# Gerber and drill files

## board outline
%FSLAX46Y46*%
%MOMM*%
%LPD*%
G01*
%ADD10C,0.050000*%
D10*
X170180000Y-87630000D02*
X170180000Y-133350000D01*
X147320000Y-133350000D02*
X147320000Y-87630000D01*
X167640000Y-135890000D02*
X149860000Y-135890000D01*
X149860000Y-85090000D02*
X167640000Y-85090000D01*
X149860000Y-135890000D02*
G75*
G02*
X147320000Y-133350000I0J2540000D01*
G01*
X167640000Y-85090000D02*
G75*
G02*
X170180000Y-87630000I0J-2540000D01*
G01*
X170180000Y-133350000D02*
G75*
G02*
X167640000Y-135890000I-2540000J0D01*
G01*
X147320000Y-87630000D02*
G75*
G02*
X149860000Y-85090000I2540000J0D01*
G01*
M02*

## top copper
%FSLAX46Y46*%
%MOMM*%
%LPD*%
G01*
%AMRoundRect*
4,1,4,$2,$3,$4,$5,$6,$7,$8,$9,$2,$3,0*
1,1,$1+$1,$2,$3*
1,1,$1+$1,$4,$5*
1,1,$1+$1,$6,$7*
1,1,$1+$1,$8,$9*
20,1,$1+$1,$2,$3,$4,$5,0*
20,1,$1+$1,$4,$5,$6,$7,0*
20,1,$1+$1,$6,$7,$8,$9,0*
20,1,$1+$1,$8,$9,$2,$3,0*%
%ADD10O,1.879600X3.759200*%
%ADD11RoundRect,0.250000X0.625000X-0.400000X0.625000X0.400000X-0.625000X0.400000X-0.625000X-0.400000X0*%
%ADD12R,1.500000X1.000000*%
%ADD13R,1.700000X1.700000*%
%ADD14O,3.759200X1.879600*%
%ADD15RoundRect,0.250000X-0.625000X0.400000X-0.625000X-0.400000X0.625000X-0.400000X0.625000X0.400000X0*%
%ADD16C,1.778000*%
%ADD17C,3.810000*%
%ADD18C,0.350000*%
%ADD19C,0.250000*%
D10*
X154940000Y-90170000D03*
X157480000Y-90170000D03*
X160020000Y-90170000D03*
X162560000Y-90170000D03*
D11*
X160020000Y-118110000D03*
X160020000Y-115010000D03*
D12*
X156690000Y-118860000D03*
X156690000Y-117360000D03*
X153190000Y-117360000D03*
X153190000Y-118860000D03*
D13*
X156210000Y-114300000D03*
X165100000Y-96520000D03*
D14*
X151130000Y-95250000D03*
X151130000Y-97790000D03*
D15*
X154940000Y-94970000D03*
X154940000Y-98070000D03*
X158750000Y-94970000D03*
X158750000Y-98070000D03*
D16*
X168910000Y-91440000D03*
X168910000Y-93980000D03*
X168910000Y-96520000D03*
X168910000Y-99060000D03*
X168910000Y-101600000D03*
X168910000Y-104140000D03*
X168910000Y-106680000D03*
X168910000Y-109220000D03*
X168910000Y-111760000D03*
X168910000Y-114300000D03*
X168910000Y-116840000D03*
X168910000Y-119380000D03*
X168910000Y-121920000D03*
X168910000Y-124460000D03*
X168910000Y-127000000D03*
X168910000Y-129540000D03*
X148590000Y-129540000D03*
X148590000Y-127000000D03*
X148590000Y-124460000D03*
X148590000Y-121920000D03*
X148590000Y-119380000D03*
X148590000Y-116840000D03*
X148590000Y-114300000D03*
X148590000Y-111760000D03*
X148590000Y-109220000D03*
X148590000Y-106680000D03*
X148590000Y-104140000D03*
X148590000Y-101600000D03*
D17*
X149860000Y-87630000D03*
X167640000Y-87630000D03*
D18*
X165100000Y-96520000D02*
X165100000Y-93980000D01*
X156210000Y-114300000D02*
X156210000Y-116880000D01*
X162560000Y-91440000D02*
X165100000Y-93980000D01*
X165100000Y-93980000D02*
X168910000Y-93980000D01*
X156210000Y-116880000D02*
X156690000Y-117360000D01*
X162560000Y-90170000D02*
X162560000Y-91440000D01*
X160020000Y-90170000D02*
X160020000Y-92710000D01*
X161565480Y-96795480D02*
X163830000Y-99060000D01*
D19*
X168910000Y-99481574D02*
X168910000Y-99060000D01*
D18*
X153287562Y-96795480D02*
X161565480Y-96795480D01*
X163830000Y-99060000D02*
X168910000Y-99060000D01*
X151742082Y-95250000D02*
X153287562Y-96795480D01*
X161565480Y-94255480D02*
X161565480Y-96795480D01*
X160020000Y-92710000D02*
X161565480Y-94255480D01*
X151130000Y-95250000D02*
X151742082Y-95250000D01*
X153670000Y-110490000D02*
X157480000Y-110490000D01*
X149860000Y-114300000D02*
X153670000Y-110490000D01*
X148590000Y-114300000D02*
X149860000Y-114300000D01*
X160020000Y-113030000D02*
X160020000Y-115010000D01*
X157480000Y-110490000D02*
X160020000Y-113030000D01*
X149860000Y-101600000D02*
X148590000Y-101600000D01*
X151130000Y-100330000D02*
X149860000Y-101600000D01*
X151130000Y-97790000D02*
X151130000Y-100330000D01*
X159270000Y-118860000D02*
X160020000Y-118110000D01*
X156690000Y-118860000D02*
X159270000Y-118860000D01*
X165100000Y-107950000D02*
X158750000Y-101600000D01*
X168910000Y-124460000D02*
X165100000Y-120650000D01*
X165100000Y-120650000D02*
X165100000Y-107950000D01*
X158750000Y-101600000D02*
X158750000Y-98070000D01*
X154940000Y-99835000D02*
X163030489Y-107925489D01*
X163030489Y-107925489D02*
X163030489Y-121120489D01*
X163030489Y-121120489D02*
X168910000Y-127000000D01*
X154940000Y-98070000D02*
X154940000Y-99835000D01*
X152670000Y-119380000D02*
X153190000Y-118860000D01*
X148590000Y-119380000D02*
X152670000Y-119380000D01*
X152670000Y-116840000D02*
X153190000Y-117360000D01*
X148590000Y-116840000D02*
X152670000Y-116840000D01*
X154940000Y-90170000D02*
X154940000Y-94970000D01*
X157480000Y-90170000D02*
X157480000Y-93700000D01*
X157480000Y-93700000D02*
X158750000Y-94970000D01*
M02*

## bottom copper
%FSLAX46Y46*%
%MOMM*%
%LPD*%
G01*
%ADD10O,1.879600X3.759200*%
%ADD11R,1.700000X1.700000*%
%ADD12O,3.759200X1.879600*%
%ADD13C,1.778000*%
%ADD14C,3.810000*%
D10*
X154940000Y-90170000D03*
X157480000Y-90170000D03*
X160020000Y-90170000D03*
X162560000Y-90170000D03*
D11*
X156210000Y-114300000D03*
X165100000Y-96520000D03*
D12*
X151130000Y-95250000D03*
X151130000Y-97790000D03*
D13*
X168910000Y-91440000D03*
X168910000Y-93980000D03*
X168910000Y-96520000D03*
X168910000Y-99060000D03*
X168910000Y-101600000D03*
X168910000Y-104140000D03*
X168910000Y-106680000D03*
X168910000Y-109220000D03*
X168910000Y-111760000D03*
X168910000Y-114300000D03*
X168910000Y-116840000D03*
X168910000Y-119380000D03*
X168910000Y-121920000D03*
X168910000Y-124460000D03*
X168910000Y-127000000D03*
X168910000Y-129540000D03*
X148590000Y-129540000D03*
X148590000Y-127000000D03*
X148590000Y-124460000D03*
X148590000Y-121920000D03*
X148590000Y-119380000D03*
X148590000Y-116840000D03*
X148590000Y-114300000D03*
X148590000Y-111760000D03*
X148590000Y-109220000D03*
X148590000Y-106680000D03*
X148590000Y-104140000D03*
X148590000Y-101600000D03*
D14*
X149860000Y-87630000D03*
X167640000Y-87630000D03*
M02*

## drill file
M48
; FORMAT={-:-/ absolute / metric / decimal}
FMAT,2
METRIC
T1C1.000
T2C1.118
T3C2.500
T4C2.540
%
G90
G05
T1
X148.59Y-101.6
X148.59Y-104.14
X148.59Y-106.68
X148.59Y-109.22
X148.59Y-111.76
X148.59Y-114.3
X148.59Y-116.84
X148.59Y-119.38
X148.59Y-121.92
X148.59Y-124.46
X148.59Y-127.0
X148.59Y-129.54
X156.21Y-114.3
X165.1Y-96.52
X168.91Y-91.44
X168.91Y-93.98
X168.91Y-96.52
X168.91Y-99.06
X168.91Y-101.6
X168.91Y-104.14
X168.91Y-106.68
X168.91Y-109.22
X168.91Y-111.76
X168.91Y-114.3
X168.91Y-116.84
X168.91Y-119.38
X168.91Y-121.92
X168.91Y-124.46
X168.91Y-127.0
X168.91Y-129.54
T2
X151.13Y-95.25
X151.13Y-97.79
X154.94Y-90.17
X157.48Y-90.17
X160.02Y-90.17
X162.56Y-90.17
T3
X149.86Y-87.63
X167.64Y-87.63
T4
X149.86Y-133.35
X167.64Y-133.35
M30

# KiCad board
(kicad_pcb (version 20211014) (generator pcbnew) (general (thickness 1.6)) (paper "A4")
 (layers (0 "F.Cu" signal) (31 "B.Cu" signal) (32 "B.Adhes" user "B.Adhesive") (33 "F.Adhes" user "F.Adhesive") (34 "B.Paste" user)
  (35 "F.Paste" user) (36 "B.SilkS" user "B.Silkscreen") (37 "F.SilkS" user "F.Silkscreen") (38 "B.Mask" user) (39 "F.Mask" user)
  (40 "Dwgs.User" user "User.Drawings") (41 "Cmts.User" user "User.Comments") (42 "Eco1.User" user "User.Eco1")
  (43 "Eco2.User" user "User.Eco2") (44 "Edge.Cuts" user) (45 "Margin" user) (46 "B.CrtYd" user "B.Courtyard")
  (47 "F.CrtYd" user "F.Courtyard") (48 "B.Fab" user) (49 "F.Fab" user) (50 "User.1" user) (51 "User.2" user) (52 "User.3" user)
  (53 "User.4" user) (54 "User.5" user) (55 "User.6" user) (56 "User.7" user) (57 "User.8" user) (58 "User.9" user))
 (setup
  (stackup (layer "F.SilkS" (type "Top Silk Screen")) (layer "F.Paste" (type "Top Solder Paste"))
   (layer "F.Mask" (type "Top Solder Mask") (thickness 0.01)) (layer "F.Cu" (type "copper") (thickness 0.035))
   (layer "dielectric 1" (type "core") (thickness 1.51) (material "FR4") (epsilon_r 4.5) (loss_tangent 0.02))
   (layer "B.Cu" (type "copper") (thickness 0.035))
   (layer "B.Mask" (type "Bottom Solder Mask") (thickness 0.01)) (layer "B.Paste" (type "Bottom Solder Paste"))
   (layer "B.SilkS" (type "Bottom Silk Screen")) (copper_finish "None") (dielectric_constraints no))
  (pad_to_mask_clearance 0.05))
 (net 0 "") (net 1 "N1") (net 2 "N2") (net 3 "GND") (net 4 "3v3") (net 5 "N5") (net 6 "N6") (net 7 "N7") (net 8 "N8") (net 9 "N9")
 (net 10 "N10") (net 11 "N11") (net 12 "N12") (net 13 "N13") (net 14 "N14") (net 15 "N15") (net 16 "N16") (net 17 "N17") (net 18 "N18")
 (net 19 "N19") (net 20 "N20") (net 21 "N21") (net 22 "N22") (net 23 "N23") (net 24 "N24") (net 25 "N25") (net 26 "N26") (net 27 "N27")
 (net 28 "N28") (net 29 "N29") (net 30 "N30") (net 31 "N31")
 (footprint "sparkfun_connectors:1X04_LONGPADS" (layer "F.Cu") (at 154.94 90.17)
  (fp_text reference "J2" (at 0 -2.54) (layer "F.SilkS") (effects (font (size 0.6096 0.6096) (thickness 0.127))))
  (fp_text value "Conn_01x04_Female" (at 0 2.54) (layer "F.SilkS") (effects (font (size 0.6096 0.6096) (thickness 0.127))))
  (pad "1" thru_hole oval locked (at 0 0 180) (size 1.8796 3.7592) (drill 1.1176) (layers *.Cu *.Mask) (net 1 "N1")
   (solder_mask_margin 0.1016))
  (pad "2" thru_hole oval locked (at 2.54 0 180) (size 1.8796 3.7592) (drill 1.1176) (layers *.Cu *.Mask) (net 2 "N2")
   (solder_mask_margin 0.1016))
  (pad "3" thru_hole oval locked (at 5.08 0 180) (size 1.8796 3.7592) (drill 1.1176) (layers *.Cu *.Mask) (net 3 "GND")
   (solder_mask_margin 0.1016))
  (pad "4" thru_hole oval locked (at 7.62 0 180) (size 1.8796 3.7592) (drill 1.1176) (layers *.Cu *.Mask) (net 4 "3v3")
   (solder_mask_margin 0.1016)))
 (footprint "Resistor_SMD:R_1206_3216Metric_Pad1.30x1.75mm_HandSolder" (layer "F.Cu") (at 160.02 116.56 90)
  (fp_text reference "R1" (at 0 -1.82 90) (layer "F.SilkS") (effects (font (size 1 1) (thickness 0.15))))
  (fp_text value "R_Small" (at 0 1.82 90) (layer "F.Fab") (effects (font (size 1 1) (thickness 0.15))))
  (pad "1" smd roundrect (at -1.55 0 90) (size 1.3 1.75) (layers "F.Cu" "F.Paste" "F.Mask") (roundrect_rratio 0.192308) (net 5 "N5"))
  (pad "2" smd roundrect (at 1.55 0 90) (size 1.3 1.75) (layers "F.Cu" "F.Paste" "F.Mask") (roundrect_rratio 0.192308) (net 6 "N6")))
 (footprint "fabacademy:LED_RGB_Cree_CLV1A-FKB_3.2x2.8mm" (layer "F.Cu") (at 154.94 118.11 180)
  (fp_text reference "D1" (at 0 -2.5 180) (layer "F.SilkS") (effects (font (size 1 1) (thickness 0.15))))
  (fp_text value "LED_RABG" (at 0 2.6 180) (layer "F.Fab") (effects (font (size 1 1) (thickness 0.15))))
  (pad "1" smd rect locked (at -1.75 -0.75) (size 1.5 1) (layers "F.Cu" "F.Paste" "F.Mask") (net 5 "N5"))
  (pad "2" smd rect locked (at -1.75 0.75) (size 1.5 1) (layers "F.Cu" "F.Paste" "F.Mask") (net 4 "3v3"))
  (pad "3" smd rect locked (at 1.75 0.75) (size 1.5 1) (layers "F.Cu" "F.Paste" "F.Mask") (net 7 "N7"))
  (pad "4" smd rect locked (at 1.75 -0.75) (size 1.5 1) (layers "F.Cu" "F.Paste" "F.Mask") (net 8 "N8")))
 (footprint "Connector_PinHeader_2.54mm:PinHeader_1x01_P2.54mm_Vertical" (layer "F.Cu") (at 156.21 114.3)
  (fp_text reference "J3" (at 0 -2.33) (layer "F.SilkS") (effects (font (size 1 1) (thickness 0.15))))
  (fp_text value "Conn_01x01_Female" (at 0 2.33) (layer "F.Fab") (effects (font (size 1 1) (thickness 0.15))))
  (pad "1" thru_hole rect (at 0 0) (size 1.7 1.7) (drill 1) (layers *.Cu *.Mask) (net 4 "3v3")))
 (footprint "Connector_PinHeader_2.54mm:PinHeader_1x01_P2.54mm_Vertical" (layer "F.Cu") (at 165.1 96.52)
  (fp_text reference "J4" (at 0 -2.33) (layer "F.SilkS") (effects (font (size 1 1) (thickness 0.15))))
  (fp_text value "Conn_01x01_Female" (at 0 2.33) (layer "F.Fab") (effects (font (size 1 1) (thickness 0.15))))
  (pad "1" thru_hole rect (at 0 0) (size 1.7 1.7) (drill 1) (layers *.Cu *.Mask) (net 4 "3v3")))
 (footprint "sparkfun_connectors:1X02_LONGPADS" (layer "F.Cu") (at 151.13 95.25 -90)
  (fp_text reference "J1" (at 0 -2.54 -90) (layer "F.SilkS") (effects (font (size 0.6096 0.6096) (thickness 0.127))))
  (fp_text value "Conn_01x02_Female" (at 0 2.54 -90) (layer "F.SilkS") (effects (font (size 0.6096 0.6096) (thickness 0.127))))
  (pad "1" thru_hole oval locked (at 0 0 90) (size 1.8796 3.7592) (drill 1.1176) (layers *.Cu *.Mask) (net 3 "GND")
   (solder_mask_margin 0.1016))
  (pad "2" thru_hole oval locked (at 2.54 0 90) (size 1.8796 3.7592) (drill 1.1176) (layers *.Cu *.Mask) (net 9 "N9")
   (solder_mask_margin 0.1016)))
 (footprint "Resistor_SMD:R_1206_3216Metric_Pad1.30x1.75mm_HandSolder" (layer "F.Cu") (at 154.94 96.52 -90)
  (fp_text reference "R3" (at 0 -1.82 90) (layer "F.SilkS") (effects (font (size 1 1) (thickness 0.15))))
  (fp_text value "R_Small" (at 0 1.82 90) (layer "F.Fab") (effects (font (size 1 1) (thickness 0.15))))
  (pad "1" smd roundrect (at -1.55 0 270) (size 1.3 1.75) (layers "F.Cu" "F.Paste" "F.Mask") (roundrect_rratio 0.192308) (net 1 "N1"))
  (pad "2" smd roundrect (at 1.55 0 270) (size 1.3 1.75) (layers "F.Cu" "F.Paste" "F.Mask") (roundrect_rratio 0.192308) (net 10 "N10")))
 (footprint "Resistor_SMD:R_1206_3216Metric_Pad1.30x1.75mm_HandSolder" (layer "F.Cu") (at 158.75 96.52 -90)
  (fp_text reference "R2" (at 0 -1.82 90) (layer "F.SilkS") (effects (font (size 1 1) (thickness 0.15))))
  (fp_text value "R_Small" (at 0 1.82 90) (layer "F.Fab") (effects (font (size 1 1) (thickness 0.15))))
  (pad "1" smd roundrect (at -1.55 0 270) (size 1.3 1.75) (layers "F.Cu" "F.Paste" "F.Mask") (roundrect_rratio 0.192308) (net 2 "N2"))
  (pad "2" smd roundrect (at 1.55 0 270) (size 1.3 1.75) (layers "F.Cu" "F.Paste" "F.Mask") (roundrect_rratio 0.192308) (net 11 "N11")))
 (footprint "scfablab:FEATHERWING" (layer "B.Cu") (at 170.18 85.09 -90)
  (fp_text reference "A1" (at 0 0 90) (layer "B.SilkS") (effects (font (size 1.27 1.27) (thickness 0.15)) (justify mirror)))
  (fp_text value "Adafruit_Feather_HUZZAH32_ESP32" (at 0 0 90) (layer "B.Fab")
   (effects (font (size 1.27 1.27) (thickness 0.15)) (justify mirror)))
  (fp_line (start 2.54 0) (end 48.26 0) (layer "Edge.Cuts") (width 0.05))
  (fp_line (start 48.26 22.86) (end 2.54 22.86) (layer "Edge.Cuts") (width 0.05))
  (fp_line (start 50.8 2.54) (end 50.8 20.32) (layer "Edge.Cuts") (width 0.05))
  (fp_line (start 0 20.32) (end 0 2.54) (layer "Edge.Cuts") (width 0.05))
  (fp_arc (start 50.8 20.32) (mid 50.056051 22.116051) (end 48.26 22.86) (layer "Edge.Cuts") (width 0.05))
  (fp_arc (start 0 2.54) (mid 0.743949 0.743949) (end 2.54 0) (layer "Edge.Cuts") (width 0.05))
  (fp_arc (start 48.26 0) (mid 50.056051 0.743949) (end 50.8 2.54) (layer "Edge.Cuts") (width 0.05))
  (fp_arc (start 2.54 22.86) (mid 0.743949 22.116051) (end 0 20.32) (layer "Edge.Cuts") (width 0.05))
  (pad "" np_thru_hole circle (at 48.26 20.32 270) (size 2.54 2.54) (drill 2.54) (layers *.Cu *.Mask))
  (pad "" np_thru_hole circle (at 48.26 2.54 270) (size 2.54 2.54) (drill 2.54) (layers *.Cu *.Mask))
  (pad "1" thru_hole circle (at 6.35 1.27 270) (size 1.778 1.778) (drill 1) (layers *.Cu *.Mask) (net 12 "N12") (solder_mask_margin 0.1016))
  (pad "2" thru_hole circle (at 8.89 1.27 270) (size 1.778 1.778) (drill 1) (layers *.Cu *.Mask) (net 4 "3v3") (solder_mask_margin 0.1016))
  (pad "3" thru_hole circle (at 11.43 1.27 270) (size 1.778 1.778) (drill 1) (layers *.Cu *.Mask) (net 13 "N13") (solder_mask_margin 0.1016))
  (pad "4" thru_hole circle (at 13.97 1.27 270) (size 1.778 1.778) (drill 1) (layers *.Cu *.Mask) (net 3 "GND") (solder_mask_margin 0.1016))
  (pad "5" thru_hole circle (at 16.51 1.27 270) (size 1.778 1.778) (drill 1) (layers *.Cu *.Mask) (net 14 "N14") (solder_mask_margin 0.1016))
  (pad "6" thru_hole circle (at 19.05 1.27 270) (size 1.778 1.778) (drill 1) (layers *.Cu *.Mask) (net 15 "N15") (solder_mask_margin 0.1016))
  (pad "7" thru_hole circle (at 21.59 1.27 270) (size 1.778 1.778) (drill 1) (layers *.Cu *.Mask) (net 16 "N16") (solder_mask_margin 0.1016))
  (pad "8" thru_hole circle (at 24.13 1.27 270) (size 1.778 1.778) (drill 1) (layers *.Cu *.Mask) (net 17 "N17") (solder_mask_margin 0.1016))
  (pad "9" thru_hole circle (at 26.67 1.27 270) (size 1.778 1.778) (drill 1) (layers *.Cu *.Mask) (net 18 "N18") (solder_mask_margin 0.1016))
  (pad "10" thru_hole circle (at 29.21 1.27 270) (size 1.778 1.778) (drill 1) (layers *.Cu *.Mask) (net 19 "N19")
   (solder_mask_margin 0.1016))
  (pad "11" thru_hole circle (at 31.75 1.27 270) (size 1.778 1.778) (drill 1) (layers *.Cu *.Mask) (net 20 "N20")
   (solder_mask_margin 0.1016))
  (pad "12" thru_hole circle (at 34.29 1.27 270) (size 1.778 1.778) (drill 1) (layers *.Cu *.Mask) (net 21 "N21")
   (solder_mask_margin 0.1016))
  (pad "13" thru_hole circle (at 36.83 1.27 270) (size 1.778 1.778) (drill 1) (layers *.Cu *.Mask) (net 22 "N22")
   (solder_mask_margin 0.1016))
  (pad "14" thru_hole circle (at 39.37 1.27 270) (size 1.778 1.778) (drill 1) (layers *.Cu *.Mask) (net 11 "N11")
   (solder_mask_margin 0.1016))
  (pad "15" thru_hole circle (at 41.91 1.27 270) (size 1.778 1.778) (drill 1) (layers *.Cu *.Mask) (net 10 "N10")
   (solder_mask_margin 0.1016))
  (pad "16" thru_hole circle (at 44.45 1.27 270) (size 1.778 1.778) (drill 1) (layers *.Cu *.Mask) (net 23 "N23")
   (solder_mask_margin 0.1016))
  (pad "17" thru_hole circle (at 44.45 21.59 270) (size 1.778 1.778) (drill 1) (layers *.Cu *.Mask) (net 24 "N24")
   (solder_mask_margin 0.1016))
  (pad "18" thru_hole circle (at 41.91 21.59 270) (size 1.778 1.778) (drill 1) (layers *.Cu *.Mask) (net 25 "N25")
   (solder_mask_margin 0.1016))
  (pad "19" thru_hole circle (at 39.37 21.59 270) (size 1.778 1.778) (drill 1) (layers *.Cu *.Mask) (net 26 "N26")
   (solder_mask_margin 0.1016))
  (pad "20" thru_hole circle (at 36.83 21.59 270) (size 1.778 1.778) (drill 1) (layers *.Cu *.Mask) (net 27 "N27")
   (solder_mask_margin 0.1016))
  (pad "21" thru_hole circle (at 34.29 21.59 270) (size 1.778 1.778) (drill 1) (layers *.Cu *.Mask) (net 8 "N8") (solder_mask_margin 0.1016))
  (pad "22" thru_hole circle (at 31.75 21.59 270) (size 1.778 1.778) (drill 1) (layers *.Cu *.Mask) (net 7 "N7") (solder_mask_margin 0.1016))
  (pad "23" thru_hole circle (at 29.21 21.59 270) (size 1.778 1.778) (drill 1) (layers *.Cu *.Mask) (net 6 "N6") (solder_mask_margin 0.1016))
  (pad "24" thru_hole circle (at 26.67 21.59 270) (size 1.778 1.778) (drill 1) (layers *.Cu *.Mask) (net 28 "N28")
   (solder_mask_margin 0.1016))
  (pad "25" thru_hole circle (at 24.13 21.59 270) (size 1.778 1.778) (drill 1) (layers *.Cu *.Mask) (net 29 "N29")
   (solder_mask_margin 0.1016))
  (pad "26" thru_hole circle (at 21.59 21.59 270) (size 1.778 1.778) (drill 1) (layers *.Cu *.Mask) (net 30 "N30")
   (solder_mask_margin 0.1016))
  (pad "27" thru_hole circle (at 19.05 21.59 270) (size 1.778 1.778) (drill 1) (layers *.Cu *.Mask) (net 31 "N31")
   (solder_mask_margin 0.1016))
  (pad "28" thru_hole circle (at 16.51 21.59 270) (size 1.778 1.778) (drill 1) (layers *.Cu *.Mask) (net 9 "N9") (solder_mask_margin 0.1016))
  (pad "P$1" thru_hole circle (at 2.54 20.32 270) (size 3.81 3.81) (drill 2.5) (layers *.Cu *.Mask) (solder_mask_margin 0.1016))
  (pad "P$2" thru_hole circle (at 2.54 2.54 270) (size 3.81 3.81) (drill 2.5) (layers *.Cu *.Mask) (solder_mask_margin 0.1016)))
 (segment (start 165.1 96.52) (end 165.1 93.98) (width 0.35) (layer "F.Cu") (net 4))
 (segment (start 156.21 114.3) (end 156.21 116.88) (width 0.35) (layer "F.Cu") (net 4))
 (segment (start 162.56 91.44) (end 165.1 93.98) (width 0.35) (layer "F.Cu") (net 4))
 (segment (start 165.1 93.98) (end 168.91 93.98) (width 0.35) (layer "F.Cu") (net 4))
 (segment (start 156.21 116.88) (end 156.69 117.36) (width 0.35) (layer "F.Cu") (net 4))
 (segment (start 162.56 90.17) (end 162.56 91.44) (width 0.35) (layer "F.Cu") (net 4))
 (segment (start 160.02 90.17) (end 160.02 92.71) (width 0.35) (layer "F.Cu") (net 3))
 (segment (start 161.56548 96.79548) (end 163.83 99.06) (width 0.35) (layer "F.Cu") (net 3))
 (segment (start 168.91 99.481574) (end 168.91 99.06) (width 0.25) (layer "F.Cu") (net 3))
 (segment (start 153.287562 96.79548) (end 161.56548 96.79548) (width 0.35) (layer "F.Cu") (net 3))
 (segment (start 163.83 99.06) (end 168.91 99.06) (width 0.35) (layer "F.Cu") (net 3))
 (segment (start 151.742082 95.25) (end 153.287562 96.79548) (width 0.35) (layer "F.Cu") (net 3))
 (segment (start 161.56548 94.25548) (end 161.56548 96.79548) (width 0.35) (layer "F.Cu") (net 3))
 (segment (start 160.02 92.71) (end 161.56548 94.25548) (width 0.35) (layer "F.Cu") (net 3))
 (segment (start 151.13 95.25) (end 151.742082 95.25) (width 0.35) (layer "F.Cu") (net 3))
 (segment (start 153.67 110.49) (end 157.48 110.49) (width 0.35) (layer "F.Cu") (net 6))
 (segment (start 149.86 114.3) (end 153.67 110.49) (width 0.35) (layer "F.Cu") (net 6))
 (segment (start 148.59 114.3) (end 149.86 114.3) (width 0.35) (layer "F.Cu") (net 6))
 (segment (start 160.02 113.03) (end 160.02 115.01) (width 0.35) (layer "F.Cu") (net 6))
 (segment (start 157.48 110.49) (end 160.02 113.03) (width 0.35) (layer "F.Cu") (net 6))
 (segment (start 149.86 101.6) (end 148.59 101.6) (width 0.35) (layer "F.Cu") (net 9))
 (segment (start 151.13 100.33) (end 149.86 101.6) (width 0.35) (layer "F.Cu") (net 9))
 (segment (start 151.13 97.79) (end 151.13 100.33) (width 0.35) (layer "F.Cu") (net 9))
 (segment (start 159.27 118.86) (end 160.02 118.11) (width 0.35) (layer "F.Cu") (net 5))
 (segment (start 156.69 118.86) (end 159.27 118.86) (width 0.35) (layer "F.Cu") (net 5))
 (segment (start 165.1 107.95) (end 158.75 101.6) (width 0.35) (layer "F.Cu") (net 11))
 (segment (start 168.91 124.46) (end 165.1 120.65) (width 0.35) (layer "F.Cu") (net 11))
 (segment (start 165.1 120.65) (end 165.1 107.95) (width 0.35) (layer "F.Cu") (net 11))
 (segment (start 158.75 101.6) (end 158.75 98.07) (width 0.35) (layer "F.Cu") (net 11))
 (segment (start 154.94 99.835) (end 163.030489 107.925489) (width 0.35) (layer "F.Cu") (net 10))
 (segment (start 163.030489 107.925489) (end 163.030489 121.120489) (width 0.35) (layer "F.Cu") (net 10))
 (segment (start 163.030489 121.120489) (end 168.91 127) (width 0.35) (layer "F.Cu") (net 10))
 (segment (start 154.94 98.07) (end 154.94 99.835) (width 0.35) (layer "F.Cu") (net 10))
 (segment (start 152.67 119.38) (end 153.19 118.86) (width 0.35) (layer "F.Cu") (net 8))
 (segment (start 148.59 119.38) (end 152.67 119.38) (width 0.35) (layer "F.Cu") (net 8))
 (segment (start 152.67 116.84) (end 153.19 117.36) (width 0.35) (layer "F.Cu") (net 7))
 (segment (start 148.59 116.84) (end 152.67 116.84) (width 0.35) (layer "F.Cu") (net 7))
 (segment (start 154.94 90.17) (end 154.94 94.97) (width 0.35) (layer "F.Cu") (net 1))
 (segment (start 157.48 90.17) (end 157.48 93.7) (width 0.35) (layer "F.Cu") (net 2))
 (segment (start 157.48 93.7) (end 158.75 94.97) (width 0.35) (layer "F.Cu") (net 2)))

